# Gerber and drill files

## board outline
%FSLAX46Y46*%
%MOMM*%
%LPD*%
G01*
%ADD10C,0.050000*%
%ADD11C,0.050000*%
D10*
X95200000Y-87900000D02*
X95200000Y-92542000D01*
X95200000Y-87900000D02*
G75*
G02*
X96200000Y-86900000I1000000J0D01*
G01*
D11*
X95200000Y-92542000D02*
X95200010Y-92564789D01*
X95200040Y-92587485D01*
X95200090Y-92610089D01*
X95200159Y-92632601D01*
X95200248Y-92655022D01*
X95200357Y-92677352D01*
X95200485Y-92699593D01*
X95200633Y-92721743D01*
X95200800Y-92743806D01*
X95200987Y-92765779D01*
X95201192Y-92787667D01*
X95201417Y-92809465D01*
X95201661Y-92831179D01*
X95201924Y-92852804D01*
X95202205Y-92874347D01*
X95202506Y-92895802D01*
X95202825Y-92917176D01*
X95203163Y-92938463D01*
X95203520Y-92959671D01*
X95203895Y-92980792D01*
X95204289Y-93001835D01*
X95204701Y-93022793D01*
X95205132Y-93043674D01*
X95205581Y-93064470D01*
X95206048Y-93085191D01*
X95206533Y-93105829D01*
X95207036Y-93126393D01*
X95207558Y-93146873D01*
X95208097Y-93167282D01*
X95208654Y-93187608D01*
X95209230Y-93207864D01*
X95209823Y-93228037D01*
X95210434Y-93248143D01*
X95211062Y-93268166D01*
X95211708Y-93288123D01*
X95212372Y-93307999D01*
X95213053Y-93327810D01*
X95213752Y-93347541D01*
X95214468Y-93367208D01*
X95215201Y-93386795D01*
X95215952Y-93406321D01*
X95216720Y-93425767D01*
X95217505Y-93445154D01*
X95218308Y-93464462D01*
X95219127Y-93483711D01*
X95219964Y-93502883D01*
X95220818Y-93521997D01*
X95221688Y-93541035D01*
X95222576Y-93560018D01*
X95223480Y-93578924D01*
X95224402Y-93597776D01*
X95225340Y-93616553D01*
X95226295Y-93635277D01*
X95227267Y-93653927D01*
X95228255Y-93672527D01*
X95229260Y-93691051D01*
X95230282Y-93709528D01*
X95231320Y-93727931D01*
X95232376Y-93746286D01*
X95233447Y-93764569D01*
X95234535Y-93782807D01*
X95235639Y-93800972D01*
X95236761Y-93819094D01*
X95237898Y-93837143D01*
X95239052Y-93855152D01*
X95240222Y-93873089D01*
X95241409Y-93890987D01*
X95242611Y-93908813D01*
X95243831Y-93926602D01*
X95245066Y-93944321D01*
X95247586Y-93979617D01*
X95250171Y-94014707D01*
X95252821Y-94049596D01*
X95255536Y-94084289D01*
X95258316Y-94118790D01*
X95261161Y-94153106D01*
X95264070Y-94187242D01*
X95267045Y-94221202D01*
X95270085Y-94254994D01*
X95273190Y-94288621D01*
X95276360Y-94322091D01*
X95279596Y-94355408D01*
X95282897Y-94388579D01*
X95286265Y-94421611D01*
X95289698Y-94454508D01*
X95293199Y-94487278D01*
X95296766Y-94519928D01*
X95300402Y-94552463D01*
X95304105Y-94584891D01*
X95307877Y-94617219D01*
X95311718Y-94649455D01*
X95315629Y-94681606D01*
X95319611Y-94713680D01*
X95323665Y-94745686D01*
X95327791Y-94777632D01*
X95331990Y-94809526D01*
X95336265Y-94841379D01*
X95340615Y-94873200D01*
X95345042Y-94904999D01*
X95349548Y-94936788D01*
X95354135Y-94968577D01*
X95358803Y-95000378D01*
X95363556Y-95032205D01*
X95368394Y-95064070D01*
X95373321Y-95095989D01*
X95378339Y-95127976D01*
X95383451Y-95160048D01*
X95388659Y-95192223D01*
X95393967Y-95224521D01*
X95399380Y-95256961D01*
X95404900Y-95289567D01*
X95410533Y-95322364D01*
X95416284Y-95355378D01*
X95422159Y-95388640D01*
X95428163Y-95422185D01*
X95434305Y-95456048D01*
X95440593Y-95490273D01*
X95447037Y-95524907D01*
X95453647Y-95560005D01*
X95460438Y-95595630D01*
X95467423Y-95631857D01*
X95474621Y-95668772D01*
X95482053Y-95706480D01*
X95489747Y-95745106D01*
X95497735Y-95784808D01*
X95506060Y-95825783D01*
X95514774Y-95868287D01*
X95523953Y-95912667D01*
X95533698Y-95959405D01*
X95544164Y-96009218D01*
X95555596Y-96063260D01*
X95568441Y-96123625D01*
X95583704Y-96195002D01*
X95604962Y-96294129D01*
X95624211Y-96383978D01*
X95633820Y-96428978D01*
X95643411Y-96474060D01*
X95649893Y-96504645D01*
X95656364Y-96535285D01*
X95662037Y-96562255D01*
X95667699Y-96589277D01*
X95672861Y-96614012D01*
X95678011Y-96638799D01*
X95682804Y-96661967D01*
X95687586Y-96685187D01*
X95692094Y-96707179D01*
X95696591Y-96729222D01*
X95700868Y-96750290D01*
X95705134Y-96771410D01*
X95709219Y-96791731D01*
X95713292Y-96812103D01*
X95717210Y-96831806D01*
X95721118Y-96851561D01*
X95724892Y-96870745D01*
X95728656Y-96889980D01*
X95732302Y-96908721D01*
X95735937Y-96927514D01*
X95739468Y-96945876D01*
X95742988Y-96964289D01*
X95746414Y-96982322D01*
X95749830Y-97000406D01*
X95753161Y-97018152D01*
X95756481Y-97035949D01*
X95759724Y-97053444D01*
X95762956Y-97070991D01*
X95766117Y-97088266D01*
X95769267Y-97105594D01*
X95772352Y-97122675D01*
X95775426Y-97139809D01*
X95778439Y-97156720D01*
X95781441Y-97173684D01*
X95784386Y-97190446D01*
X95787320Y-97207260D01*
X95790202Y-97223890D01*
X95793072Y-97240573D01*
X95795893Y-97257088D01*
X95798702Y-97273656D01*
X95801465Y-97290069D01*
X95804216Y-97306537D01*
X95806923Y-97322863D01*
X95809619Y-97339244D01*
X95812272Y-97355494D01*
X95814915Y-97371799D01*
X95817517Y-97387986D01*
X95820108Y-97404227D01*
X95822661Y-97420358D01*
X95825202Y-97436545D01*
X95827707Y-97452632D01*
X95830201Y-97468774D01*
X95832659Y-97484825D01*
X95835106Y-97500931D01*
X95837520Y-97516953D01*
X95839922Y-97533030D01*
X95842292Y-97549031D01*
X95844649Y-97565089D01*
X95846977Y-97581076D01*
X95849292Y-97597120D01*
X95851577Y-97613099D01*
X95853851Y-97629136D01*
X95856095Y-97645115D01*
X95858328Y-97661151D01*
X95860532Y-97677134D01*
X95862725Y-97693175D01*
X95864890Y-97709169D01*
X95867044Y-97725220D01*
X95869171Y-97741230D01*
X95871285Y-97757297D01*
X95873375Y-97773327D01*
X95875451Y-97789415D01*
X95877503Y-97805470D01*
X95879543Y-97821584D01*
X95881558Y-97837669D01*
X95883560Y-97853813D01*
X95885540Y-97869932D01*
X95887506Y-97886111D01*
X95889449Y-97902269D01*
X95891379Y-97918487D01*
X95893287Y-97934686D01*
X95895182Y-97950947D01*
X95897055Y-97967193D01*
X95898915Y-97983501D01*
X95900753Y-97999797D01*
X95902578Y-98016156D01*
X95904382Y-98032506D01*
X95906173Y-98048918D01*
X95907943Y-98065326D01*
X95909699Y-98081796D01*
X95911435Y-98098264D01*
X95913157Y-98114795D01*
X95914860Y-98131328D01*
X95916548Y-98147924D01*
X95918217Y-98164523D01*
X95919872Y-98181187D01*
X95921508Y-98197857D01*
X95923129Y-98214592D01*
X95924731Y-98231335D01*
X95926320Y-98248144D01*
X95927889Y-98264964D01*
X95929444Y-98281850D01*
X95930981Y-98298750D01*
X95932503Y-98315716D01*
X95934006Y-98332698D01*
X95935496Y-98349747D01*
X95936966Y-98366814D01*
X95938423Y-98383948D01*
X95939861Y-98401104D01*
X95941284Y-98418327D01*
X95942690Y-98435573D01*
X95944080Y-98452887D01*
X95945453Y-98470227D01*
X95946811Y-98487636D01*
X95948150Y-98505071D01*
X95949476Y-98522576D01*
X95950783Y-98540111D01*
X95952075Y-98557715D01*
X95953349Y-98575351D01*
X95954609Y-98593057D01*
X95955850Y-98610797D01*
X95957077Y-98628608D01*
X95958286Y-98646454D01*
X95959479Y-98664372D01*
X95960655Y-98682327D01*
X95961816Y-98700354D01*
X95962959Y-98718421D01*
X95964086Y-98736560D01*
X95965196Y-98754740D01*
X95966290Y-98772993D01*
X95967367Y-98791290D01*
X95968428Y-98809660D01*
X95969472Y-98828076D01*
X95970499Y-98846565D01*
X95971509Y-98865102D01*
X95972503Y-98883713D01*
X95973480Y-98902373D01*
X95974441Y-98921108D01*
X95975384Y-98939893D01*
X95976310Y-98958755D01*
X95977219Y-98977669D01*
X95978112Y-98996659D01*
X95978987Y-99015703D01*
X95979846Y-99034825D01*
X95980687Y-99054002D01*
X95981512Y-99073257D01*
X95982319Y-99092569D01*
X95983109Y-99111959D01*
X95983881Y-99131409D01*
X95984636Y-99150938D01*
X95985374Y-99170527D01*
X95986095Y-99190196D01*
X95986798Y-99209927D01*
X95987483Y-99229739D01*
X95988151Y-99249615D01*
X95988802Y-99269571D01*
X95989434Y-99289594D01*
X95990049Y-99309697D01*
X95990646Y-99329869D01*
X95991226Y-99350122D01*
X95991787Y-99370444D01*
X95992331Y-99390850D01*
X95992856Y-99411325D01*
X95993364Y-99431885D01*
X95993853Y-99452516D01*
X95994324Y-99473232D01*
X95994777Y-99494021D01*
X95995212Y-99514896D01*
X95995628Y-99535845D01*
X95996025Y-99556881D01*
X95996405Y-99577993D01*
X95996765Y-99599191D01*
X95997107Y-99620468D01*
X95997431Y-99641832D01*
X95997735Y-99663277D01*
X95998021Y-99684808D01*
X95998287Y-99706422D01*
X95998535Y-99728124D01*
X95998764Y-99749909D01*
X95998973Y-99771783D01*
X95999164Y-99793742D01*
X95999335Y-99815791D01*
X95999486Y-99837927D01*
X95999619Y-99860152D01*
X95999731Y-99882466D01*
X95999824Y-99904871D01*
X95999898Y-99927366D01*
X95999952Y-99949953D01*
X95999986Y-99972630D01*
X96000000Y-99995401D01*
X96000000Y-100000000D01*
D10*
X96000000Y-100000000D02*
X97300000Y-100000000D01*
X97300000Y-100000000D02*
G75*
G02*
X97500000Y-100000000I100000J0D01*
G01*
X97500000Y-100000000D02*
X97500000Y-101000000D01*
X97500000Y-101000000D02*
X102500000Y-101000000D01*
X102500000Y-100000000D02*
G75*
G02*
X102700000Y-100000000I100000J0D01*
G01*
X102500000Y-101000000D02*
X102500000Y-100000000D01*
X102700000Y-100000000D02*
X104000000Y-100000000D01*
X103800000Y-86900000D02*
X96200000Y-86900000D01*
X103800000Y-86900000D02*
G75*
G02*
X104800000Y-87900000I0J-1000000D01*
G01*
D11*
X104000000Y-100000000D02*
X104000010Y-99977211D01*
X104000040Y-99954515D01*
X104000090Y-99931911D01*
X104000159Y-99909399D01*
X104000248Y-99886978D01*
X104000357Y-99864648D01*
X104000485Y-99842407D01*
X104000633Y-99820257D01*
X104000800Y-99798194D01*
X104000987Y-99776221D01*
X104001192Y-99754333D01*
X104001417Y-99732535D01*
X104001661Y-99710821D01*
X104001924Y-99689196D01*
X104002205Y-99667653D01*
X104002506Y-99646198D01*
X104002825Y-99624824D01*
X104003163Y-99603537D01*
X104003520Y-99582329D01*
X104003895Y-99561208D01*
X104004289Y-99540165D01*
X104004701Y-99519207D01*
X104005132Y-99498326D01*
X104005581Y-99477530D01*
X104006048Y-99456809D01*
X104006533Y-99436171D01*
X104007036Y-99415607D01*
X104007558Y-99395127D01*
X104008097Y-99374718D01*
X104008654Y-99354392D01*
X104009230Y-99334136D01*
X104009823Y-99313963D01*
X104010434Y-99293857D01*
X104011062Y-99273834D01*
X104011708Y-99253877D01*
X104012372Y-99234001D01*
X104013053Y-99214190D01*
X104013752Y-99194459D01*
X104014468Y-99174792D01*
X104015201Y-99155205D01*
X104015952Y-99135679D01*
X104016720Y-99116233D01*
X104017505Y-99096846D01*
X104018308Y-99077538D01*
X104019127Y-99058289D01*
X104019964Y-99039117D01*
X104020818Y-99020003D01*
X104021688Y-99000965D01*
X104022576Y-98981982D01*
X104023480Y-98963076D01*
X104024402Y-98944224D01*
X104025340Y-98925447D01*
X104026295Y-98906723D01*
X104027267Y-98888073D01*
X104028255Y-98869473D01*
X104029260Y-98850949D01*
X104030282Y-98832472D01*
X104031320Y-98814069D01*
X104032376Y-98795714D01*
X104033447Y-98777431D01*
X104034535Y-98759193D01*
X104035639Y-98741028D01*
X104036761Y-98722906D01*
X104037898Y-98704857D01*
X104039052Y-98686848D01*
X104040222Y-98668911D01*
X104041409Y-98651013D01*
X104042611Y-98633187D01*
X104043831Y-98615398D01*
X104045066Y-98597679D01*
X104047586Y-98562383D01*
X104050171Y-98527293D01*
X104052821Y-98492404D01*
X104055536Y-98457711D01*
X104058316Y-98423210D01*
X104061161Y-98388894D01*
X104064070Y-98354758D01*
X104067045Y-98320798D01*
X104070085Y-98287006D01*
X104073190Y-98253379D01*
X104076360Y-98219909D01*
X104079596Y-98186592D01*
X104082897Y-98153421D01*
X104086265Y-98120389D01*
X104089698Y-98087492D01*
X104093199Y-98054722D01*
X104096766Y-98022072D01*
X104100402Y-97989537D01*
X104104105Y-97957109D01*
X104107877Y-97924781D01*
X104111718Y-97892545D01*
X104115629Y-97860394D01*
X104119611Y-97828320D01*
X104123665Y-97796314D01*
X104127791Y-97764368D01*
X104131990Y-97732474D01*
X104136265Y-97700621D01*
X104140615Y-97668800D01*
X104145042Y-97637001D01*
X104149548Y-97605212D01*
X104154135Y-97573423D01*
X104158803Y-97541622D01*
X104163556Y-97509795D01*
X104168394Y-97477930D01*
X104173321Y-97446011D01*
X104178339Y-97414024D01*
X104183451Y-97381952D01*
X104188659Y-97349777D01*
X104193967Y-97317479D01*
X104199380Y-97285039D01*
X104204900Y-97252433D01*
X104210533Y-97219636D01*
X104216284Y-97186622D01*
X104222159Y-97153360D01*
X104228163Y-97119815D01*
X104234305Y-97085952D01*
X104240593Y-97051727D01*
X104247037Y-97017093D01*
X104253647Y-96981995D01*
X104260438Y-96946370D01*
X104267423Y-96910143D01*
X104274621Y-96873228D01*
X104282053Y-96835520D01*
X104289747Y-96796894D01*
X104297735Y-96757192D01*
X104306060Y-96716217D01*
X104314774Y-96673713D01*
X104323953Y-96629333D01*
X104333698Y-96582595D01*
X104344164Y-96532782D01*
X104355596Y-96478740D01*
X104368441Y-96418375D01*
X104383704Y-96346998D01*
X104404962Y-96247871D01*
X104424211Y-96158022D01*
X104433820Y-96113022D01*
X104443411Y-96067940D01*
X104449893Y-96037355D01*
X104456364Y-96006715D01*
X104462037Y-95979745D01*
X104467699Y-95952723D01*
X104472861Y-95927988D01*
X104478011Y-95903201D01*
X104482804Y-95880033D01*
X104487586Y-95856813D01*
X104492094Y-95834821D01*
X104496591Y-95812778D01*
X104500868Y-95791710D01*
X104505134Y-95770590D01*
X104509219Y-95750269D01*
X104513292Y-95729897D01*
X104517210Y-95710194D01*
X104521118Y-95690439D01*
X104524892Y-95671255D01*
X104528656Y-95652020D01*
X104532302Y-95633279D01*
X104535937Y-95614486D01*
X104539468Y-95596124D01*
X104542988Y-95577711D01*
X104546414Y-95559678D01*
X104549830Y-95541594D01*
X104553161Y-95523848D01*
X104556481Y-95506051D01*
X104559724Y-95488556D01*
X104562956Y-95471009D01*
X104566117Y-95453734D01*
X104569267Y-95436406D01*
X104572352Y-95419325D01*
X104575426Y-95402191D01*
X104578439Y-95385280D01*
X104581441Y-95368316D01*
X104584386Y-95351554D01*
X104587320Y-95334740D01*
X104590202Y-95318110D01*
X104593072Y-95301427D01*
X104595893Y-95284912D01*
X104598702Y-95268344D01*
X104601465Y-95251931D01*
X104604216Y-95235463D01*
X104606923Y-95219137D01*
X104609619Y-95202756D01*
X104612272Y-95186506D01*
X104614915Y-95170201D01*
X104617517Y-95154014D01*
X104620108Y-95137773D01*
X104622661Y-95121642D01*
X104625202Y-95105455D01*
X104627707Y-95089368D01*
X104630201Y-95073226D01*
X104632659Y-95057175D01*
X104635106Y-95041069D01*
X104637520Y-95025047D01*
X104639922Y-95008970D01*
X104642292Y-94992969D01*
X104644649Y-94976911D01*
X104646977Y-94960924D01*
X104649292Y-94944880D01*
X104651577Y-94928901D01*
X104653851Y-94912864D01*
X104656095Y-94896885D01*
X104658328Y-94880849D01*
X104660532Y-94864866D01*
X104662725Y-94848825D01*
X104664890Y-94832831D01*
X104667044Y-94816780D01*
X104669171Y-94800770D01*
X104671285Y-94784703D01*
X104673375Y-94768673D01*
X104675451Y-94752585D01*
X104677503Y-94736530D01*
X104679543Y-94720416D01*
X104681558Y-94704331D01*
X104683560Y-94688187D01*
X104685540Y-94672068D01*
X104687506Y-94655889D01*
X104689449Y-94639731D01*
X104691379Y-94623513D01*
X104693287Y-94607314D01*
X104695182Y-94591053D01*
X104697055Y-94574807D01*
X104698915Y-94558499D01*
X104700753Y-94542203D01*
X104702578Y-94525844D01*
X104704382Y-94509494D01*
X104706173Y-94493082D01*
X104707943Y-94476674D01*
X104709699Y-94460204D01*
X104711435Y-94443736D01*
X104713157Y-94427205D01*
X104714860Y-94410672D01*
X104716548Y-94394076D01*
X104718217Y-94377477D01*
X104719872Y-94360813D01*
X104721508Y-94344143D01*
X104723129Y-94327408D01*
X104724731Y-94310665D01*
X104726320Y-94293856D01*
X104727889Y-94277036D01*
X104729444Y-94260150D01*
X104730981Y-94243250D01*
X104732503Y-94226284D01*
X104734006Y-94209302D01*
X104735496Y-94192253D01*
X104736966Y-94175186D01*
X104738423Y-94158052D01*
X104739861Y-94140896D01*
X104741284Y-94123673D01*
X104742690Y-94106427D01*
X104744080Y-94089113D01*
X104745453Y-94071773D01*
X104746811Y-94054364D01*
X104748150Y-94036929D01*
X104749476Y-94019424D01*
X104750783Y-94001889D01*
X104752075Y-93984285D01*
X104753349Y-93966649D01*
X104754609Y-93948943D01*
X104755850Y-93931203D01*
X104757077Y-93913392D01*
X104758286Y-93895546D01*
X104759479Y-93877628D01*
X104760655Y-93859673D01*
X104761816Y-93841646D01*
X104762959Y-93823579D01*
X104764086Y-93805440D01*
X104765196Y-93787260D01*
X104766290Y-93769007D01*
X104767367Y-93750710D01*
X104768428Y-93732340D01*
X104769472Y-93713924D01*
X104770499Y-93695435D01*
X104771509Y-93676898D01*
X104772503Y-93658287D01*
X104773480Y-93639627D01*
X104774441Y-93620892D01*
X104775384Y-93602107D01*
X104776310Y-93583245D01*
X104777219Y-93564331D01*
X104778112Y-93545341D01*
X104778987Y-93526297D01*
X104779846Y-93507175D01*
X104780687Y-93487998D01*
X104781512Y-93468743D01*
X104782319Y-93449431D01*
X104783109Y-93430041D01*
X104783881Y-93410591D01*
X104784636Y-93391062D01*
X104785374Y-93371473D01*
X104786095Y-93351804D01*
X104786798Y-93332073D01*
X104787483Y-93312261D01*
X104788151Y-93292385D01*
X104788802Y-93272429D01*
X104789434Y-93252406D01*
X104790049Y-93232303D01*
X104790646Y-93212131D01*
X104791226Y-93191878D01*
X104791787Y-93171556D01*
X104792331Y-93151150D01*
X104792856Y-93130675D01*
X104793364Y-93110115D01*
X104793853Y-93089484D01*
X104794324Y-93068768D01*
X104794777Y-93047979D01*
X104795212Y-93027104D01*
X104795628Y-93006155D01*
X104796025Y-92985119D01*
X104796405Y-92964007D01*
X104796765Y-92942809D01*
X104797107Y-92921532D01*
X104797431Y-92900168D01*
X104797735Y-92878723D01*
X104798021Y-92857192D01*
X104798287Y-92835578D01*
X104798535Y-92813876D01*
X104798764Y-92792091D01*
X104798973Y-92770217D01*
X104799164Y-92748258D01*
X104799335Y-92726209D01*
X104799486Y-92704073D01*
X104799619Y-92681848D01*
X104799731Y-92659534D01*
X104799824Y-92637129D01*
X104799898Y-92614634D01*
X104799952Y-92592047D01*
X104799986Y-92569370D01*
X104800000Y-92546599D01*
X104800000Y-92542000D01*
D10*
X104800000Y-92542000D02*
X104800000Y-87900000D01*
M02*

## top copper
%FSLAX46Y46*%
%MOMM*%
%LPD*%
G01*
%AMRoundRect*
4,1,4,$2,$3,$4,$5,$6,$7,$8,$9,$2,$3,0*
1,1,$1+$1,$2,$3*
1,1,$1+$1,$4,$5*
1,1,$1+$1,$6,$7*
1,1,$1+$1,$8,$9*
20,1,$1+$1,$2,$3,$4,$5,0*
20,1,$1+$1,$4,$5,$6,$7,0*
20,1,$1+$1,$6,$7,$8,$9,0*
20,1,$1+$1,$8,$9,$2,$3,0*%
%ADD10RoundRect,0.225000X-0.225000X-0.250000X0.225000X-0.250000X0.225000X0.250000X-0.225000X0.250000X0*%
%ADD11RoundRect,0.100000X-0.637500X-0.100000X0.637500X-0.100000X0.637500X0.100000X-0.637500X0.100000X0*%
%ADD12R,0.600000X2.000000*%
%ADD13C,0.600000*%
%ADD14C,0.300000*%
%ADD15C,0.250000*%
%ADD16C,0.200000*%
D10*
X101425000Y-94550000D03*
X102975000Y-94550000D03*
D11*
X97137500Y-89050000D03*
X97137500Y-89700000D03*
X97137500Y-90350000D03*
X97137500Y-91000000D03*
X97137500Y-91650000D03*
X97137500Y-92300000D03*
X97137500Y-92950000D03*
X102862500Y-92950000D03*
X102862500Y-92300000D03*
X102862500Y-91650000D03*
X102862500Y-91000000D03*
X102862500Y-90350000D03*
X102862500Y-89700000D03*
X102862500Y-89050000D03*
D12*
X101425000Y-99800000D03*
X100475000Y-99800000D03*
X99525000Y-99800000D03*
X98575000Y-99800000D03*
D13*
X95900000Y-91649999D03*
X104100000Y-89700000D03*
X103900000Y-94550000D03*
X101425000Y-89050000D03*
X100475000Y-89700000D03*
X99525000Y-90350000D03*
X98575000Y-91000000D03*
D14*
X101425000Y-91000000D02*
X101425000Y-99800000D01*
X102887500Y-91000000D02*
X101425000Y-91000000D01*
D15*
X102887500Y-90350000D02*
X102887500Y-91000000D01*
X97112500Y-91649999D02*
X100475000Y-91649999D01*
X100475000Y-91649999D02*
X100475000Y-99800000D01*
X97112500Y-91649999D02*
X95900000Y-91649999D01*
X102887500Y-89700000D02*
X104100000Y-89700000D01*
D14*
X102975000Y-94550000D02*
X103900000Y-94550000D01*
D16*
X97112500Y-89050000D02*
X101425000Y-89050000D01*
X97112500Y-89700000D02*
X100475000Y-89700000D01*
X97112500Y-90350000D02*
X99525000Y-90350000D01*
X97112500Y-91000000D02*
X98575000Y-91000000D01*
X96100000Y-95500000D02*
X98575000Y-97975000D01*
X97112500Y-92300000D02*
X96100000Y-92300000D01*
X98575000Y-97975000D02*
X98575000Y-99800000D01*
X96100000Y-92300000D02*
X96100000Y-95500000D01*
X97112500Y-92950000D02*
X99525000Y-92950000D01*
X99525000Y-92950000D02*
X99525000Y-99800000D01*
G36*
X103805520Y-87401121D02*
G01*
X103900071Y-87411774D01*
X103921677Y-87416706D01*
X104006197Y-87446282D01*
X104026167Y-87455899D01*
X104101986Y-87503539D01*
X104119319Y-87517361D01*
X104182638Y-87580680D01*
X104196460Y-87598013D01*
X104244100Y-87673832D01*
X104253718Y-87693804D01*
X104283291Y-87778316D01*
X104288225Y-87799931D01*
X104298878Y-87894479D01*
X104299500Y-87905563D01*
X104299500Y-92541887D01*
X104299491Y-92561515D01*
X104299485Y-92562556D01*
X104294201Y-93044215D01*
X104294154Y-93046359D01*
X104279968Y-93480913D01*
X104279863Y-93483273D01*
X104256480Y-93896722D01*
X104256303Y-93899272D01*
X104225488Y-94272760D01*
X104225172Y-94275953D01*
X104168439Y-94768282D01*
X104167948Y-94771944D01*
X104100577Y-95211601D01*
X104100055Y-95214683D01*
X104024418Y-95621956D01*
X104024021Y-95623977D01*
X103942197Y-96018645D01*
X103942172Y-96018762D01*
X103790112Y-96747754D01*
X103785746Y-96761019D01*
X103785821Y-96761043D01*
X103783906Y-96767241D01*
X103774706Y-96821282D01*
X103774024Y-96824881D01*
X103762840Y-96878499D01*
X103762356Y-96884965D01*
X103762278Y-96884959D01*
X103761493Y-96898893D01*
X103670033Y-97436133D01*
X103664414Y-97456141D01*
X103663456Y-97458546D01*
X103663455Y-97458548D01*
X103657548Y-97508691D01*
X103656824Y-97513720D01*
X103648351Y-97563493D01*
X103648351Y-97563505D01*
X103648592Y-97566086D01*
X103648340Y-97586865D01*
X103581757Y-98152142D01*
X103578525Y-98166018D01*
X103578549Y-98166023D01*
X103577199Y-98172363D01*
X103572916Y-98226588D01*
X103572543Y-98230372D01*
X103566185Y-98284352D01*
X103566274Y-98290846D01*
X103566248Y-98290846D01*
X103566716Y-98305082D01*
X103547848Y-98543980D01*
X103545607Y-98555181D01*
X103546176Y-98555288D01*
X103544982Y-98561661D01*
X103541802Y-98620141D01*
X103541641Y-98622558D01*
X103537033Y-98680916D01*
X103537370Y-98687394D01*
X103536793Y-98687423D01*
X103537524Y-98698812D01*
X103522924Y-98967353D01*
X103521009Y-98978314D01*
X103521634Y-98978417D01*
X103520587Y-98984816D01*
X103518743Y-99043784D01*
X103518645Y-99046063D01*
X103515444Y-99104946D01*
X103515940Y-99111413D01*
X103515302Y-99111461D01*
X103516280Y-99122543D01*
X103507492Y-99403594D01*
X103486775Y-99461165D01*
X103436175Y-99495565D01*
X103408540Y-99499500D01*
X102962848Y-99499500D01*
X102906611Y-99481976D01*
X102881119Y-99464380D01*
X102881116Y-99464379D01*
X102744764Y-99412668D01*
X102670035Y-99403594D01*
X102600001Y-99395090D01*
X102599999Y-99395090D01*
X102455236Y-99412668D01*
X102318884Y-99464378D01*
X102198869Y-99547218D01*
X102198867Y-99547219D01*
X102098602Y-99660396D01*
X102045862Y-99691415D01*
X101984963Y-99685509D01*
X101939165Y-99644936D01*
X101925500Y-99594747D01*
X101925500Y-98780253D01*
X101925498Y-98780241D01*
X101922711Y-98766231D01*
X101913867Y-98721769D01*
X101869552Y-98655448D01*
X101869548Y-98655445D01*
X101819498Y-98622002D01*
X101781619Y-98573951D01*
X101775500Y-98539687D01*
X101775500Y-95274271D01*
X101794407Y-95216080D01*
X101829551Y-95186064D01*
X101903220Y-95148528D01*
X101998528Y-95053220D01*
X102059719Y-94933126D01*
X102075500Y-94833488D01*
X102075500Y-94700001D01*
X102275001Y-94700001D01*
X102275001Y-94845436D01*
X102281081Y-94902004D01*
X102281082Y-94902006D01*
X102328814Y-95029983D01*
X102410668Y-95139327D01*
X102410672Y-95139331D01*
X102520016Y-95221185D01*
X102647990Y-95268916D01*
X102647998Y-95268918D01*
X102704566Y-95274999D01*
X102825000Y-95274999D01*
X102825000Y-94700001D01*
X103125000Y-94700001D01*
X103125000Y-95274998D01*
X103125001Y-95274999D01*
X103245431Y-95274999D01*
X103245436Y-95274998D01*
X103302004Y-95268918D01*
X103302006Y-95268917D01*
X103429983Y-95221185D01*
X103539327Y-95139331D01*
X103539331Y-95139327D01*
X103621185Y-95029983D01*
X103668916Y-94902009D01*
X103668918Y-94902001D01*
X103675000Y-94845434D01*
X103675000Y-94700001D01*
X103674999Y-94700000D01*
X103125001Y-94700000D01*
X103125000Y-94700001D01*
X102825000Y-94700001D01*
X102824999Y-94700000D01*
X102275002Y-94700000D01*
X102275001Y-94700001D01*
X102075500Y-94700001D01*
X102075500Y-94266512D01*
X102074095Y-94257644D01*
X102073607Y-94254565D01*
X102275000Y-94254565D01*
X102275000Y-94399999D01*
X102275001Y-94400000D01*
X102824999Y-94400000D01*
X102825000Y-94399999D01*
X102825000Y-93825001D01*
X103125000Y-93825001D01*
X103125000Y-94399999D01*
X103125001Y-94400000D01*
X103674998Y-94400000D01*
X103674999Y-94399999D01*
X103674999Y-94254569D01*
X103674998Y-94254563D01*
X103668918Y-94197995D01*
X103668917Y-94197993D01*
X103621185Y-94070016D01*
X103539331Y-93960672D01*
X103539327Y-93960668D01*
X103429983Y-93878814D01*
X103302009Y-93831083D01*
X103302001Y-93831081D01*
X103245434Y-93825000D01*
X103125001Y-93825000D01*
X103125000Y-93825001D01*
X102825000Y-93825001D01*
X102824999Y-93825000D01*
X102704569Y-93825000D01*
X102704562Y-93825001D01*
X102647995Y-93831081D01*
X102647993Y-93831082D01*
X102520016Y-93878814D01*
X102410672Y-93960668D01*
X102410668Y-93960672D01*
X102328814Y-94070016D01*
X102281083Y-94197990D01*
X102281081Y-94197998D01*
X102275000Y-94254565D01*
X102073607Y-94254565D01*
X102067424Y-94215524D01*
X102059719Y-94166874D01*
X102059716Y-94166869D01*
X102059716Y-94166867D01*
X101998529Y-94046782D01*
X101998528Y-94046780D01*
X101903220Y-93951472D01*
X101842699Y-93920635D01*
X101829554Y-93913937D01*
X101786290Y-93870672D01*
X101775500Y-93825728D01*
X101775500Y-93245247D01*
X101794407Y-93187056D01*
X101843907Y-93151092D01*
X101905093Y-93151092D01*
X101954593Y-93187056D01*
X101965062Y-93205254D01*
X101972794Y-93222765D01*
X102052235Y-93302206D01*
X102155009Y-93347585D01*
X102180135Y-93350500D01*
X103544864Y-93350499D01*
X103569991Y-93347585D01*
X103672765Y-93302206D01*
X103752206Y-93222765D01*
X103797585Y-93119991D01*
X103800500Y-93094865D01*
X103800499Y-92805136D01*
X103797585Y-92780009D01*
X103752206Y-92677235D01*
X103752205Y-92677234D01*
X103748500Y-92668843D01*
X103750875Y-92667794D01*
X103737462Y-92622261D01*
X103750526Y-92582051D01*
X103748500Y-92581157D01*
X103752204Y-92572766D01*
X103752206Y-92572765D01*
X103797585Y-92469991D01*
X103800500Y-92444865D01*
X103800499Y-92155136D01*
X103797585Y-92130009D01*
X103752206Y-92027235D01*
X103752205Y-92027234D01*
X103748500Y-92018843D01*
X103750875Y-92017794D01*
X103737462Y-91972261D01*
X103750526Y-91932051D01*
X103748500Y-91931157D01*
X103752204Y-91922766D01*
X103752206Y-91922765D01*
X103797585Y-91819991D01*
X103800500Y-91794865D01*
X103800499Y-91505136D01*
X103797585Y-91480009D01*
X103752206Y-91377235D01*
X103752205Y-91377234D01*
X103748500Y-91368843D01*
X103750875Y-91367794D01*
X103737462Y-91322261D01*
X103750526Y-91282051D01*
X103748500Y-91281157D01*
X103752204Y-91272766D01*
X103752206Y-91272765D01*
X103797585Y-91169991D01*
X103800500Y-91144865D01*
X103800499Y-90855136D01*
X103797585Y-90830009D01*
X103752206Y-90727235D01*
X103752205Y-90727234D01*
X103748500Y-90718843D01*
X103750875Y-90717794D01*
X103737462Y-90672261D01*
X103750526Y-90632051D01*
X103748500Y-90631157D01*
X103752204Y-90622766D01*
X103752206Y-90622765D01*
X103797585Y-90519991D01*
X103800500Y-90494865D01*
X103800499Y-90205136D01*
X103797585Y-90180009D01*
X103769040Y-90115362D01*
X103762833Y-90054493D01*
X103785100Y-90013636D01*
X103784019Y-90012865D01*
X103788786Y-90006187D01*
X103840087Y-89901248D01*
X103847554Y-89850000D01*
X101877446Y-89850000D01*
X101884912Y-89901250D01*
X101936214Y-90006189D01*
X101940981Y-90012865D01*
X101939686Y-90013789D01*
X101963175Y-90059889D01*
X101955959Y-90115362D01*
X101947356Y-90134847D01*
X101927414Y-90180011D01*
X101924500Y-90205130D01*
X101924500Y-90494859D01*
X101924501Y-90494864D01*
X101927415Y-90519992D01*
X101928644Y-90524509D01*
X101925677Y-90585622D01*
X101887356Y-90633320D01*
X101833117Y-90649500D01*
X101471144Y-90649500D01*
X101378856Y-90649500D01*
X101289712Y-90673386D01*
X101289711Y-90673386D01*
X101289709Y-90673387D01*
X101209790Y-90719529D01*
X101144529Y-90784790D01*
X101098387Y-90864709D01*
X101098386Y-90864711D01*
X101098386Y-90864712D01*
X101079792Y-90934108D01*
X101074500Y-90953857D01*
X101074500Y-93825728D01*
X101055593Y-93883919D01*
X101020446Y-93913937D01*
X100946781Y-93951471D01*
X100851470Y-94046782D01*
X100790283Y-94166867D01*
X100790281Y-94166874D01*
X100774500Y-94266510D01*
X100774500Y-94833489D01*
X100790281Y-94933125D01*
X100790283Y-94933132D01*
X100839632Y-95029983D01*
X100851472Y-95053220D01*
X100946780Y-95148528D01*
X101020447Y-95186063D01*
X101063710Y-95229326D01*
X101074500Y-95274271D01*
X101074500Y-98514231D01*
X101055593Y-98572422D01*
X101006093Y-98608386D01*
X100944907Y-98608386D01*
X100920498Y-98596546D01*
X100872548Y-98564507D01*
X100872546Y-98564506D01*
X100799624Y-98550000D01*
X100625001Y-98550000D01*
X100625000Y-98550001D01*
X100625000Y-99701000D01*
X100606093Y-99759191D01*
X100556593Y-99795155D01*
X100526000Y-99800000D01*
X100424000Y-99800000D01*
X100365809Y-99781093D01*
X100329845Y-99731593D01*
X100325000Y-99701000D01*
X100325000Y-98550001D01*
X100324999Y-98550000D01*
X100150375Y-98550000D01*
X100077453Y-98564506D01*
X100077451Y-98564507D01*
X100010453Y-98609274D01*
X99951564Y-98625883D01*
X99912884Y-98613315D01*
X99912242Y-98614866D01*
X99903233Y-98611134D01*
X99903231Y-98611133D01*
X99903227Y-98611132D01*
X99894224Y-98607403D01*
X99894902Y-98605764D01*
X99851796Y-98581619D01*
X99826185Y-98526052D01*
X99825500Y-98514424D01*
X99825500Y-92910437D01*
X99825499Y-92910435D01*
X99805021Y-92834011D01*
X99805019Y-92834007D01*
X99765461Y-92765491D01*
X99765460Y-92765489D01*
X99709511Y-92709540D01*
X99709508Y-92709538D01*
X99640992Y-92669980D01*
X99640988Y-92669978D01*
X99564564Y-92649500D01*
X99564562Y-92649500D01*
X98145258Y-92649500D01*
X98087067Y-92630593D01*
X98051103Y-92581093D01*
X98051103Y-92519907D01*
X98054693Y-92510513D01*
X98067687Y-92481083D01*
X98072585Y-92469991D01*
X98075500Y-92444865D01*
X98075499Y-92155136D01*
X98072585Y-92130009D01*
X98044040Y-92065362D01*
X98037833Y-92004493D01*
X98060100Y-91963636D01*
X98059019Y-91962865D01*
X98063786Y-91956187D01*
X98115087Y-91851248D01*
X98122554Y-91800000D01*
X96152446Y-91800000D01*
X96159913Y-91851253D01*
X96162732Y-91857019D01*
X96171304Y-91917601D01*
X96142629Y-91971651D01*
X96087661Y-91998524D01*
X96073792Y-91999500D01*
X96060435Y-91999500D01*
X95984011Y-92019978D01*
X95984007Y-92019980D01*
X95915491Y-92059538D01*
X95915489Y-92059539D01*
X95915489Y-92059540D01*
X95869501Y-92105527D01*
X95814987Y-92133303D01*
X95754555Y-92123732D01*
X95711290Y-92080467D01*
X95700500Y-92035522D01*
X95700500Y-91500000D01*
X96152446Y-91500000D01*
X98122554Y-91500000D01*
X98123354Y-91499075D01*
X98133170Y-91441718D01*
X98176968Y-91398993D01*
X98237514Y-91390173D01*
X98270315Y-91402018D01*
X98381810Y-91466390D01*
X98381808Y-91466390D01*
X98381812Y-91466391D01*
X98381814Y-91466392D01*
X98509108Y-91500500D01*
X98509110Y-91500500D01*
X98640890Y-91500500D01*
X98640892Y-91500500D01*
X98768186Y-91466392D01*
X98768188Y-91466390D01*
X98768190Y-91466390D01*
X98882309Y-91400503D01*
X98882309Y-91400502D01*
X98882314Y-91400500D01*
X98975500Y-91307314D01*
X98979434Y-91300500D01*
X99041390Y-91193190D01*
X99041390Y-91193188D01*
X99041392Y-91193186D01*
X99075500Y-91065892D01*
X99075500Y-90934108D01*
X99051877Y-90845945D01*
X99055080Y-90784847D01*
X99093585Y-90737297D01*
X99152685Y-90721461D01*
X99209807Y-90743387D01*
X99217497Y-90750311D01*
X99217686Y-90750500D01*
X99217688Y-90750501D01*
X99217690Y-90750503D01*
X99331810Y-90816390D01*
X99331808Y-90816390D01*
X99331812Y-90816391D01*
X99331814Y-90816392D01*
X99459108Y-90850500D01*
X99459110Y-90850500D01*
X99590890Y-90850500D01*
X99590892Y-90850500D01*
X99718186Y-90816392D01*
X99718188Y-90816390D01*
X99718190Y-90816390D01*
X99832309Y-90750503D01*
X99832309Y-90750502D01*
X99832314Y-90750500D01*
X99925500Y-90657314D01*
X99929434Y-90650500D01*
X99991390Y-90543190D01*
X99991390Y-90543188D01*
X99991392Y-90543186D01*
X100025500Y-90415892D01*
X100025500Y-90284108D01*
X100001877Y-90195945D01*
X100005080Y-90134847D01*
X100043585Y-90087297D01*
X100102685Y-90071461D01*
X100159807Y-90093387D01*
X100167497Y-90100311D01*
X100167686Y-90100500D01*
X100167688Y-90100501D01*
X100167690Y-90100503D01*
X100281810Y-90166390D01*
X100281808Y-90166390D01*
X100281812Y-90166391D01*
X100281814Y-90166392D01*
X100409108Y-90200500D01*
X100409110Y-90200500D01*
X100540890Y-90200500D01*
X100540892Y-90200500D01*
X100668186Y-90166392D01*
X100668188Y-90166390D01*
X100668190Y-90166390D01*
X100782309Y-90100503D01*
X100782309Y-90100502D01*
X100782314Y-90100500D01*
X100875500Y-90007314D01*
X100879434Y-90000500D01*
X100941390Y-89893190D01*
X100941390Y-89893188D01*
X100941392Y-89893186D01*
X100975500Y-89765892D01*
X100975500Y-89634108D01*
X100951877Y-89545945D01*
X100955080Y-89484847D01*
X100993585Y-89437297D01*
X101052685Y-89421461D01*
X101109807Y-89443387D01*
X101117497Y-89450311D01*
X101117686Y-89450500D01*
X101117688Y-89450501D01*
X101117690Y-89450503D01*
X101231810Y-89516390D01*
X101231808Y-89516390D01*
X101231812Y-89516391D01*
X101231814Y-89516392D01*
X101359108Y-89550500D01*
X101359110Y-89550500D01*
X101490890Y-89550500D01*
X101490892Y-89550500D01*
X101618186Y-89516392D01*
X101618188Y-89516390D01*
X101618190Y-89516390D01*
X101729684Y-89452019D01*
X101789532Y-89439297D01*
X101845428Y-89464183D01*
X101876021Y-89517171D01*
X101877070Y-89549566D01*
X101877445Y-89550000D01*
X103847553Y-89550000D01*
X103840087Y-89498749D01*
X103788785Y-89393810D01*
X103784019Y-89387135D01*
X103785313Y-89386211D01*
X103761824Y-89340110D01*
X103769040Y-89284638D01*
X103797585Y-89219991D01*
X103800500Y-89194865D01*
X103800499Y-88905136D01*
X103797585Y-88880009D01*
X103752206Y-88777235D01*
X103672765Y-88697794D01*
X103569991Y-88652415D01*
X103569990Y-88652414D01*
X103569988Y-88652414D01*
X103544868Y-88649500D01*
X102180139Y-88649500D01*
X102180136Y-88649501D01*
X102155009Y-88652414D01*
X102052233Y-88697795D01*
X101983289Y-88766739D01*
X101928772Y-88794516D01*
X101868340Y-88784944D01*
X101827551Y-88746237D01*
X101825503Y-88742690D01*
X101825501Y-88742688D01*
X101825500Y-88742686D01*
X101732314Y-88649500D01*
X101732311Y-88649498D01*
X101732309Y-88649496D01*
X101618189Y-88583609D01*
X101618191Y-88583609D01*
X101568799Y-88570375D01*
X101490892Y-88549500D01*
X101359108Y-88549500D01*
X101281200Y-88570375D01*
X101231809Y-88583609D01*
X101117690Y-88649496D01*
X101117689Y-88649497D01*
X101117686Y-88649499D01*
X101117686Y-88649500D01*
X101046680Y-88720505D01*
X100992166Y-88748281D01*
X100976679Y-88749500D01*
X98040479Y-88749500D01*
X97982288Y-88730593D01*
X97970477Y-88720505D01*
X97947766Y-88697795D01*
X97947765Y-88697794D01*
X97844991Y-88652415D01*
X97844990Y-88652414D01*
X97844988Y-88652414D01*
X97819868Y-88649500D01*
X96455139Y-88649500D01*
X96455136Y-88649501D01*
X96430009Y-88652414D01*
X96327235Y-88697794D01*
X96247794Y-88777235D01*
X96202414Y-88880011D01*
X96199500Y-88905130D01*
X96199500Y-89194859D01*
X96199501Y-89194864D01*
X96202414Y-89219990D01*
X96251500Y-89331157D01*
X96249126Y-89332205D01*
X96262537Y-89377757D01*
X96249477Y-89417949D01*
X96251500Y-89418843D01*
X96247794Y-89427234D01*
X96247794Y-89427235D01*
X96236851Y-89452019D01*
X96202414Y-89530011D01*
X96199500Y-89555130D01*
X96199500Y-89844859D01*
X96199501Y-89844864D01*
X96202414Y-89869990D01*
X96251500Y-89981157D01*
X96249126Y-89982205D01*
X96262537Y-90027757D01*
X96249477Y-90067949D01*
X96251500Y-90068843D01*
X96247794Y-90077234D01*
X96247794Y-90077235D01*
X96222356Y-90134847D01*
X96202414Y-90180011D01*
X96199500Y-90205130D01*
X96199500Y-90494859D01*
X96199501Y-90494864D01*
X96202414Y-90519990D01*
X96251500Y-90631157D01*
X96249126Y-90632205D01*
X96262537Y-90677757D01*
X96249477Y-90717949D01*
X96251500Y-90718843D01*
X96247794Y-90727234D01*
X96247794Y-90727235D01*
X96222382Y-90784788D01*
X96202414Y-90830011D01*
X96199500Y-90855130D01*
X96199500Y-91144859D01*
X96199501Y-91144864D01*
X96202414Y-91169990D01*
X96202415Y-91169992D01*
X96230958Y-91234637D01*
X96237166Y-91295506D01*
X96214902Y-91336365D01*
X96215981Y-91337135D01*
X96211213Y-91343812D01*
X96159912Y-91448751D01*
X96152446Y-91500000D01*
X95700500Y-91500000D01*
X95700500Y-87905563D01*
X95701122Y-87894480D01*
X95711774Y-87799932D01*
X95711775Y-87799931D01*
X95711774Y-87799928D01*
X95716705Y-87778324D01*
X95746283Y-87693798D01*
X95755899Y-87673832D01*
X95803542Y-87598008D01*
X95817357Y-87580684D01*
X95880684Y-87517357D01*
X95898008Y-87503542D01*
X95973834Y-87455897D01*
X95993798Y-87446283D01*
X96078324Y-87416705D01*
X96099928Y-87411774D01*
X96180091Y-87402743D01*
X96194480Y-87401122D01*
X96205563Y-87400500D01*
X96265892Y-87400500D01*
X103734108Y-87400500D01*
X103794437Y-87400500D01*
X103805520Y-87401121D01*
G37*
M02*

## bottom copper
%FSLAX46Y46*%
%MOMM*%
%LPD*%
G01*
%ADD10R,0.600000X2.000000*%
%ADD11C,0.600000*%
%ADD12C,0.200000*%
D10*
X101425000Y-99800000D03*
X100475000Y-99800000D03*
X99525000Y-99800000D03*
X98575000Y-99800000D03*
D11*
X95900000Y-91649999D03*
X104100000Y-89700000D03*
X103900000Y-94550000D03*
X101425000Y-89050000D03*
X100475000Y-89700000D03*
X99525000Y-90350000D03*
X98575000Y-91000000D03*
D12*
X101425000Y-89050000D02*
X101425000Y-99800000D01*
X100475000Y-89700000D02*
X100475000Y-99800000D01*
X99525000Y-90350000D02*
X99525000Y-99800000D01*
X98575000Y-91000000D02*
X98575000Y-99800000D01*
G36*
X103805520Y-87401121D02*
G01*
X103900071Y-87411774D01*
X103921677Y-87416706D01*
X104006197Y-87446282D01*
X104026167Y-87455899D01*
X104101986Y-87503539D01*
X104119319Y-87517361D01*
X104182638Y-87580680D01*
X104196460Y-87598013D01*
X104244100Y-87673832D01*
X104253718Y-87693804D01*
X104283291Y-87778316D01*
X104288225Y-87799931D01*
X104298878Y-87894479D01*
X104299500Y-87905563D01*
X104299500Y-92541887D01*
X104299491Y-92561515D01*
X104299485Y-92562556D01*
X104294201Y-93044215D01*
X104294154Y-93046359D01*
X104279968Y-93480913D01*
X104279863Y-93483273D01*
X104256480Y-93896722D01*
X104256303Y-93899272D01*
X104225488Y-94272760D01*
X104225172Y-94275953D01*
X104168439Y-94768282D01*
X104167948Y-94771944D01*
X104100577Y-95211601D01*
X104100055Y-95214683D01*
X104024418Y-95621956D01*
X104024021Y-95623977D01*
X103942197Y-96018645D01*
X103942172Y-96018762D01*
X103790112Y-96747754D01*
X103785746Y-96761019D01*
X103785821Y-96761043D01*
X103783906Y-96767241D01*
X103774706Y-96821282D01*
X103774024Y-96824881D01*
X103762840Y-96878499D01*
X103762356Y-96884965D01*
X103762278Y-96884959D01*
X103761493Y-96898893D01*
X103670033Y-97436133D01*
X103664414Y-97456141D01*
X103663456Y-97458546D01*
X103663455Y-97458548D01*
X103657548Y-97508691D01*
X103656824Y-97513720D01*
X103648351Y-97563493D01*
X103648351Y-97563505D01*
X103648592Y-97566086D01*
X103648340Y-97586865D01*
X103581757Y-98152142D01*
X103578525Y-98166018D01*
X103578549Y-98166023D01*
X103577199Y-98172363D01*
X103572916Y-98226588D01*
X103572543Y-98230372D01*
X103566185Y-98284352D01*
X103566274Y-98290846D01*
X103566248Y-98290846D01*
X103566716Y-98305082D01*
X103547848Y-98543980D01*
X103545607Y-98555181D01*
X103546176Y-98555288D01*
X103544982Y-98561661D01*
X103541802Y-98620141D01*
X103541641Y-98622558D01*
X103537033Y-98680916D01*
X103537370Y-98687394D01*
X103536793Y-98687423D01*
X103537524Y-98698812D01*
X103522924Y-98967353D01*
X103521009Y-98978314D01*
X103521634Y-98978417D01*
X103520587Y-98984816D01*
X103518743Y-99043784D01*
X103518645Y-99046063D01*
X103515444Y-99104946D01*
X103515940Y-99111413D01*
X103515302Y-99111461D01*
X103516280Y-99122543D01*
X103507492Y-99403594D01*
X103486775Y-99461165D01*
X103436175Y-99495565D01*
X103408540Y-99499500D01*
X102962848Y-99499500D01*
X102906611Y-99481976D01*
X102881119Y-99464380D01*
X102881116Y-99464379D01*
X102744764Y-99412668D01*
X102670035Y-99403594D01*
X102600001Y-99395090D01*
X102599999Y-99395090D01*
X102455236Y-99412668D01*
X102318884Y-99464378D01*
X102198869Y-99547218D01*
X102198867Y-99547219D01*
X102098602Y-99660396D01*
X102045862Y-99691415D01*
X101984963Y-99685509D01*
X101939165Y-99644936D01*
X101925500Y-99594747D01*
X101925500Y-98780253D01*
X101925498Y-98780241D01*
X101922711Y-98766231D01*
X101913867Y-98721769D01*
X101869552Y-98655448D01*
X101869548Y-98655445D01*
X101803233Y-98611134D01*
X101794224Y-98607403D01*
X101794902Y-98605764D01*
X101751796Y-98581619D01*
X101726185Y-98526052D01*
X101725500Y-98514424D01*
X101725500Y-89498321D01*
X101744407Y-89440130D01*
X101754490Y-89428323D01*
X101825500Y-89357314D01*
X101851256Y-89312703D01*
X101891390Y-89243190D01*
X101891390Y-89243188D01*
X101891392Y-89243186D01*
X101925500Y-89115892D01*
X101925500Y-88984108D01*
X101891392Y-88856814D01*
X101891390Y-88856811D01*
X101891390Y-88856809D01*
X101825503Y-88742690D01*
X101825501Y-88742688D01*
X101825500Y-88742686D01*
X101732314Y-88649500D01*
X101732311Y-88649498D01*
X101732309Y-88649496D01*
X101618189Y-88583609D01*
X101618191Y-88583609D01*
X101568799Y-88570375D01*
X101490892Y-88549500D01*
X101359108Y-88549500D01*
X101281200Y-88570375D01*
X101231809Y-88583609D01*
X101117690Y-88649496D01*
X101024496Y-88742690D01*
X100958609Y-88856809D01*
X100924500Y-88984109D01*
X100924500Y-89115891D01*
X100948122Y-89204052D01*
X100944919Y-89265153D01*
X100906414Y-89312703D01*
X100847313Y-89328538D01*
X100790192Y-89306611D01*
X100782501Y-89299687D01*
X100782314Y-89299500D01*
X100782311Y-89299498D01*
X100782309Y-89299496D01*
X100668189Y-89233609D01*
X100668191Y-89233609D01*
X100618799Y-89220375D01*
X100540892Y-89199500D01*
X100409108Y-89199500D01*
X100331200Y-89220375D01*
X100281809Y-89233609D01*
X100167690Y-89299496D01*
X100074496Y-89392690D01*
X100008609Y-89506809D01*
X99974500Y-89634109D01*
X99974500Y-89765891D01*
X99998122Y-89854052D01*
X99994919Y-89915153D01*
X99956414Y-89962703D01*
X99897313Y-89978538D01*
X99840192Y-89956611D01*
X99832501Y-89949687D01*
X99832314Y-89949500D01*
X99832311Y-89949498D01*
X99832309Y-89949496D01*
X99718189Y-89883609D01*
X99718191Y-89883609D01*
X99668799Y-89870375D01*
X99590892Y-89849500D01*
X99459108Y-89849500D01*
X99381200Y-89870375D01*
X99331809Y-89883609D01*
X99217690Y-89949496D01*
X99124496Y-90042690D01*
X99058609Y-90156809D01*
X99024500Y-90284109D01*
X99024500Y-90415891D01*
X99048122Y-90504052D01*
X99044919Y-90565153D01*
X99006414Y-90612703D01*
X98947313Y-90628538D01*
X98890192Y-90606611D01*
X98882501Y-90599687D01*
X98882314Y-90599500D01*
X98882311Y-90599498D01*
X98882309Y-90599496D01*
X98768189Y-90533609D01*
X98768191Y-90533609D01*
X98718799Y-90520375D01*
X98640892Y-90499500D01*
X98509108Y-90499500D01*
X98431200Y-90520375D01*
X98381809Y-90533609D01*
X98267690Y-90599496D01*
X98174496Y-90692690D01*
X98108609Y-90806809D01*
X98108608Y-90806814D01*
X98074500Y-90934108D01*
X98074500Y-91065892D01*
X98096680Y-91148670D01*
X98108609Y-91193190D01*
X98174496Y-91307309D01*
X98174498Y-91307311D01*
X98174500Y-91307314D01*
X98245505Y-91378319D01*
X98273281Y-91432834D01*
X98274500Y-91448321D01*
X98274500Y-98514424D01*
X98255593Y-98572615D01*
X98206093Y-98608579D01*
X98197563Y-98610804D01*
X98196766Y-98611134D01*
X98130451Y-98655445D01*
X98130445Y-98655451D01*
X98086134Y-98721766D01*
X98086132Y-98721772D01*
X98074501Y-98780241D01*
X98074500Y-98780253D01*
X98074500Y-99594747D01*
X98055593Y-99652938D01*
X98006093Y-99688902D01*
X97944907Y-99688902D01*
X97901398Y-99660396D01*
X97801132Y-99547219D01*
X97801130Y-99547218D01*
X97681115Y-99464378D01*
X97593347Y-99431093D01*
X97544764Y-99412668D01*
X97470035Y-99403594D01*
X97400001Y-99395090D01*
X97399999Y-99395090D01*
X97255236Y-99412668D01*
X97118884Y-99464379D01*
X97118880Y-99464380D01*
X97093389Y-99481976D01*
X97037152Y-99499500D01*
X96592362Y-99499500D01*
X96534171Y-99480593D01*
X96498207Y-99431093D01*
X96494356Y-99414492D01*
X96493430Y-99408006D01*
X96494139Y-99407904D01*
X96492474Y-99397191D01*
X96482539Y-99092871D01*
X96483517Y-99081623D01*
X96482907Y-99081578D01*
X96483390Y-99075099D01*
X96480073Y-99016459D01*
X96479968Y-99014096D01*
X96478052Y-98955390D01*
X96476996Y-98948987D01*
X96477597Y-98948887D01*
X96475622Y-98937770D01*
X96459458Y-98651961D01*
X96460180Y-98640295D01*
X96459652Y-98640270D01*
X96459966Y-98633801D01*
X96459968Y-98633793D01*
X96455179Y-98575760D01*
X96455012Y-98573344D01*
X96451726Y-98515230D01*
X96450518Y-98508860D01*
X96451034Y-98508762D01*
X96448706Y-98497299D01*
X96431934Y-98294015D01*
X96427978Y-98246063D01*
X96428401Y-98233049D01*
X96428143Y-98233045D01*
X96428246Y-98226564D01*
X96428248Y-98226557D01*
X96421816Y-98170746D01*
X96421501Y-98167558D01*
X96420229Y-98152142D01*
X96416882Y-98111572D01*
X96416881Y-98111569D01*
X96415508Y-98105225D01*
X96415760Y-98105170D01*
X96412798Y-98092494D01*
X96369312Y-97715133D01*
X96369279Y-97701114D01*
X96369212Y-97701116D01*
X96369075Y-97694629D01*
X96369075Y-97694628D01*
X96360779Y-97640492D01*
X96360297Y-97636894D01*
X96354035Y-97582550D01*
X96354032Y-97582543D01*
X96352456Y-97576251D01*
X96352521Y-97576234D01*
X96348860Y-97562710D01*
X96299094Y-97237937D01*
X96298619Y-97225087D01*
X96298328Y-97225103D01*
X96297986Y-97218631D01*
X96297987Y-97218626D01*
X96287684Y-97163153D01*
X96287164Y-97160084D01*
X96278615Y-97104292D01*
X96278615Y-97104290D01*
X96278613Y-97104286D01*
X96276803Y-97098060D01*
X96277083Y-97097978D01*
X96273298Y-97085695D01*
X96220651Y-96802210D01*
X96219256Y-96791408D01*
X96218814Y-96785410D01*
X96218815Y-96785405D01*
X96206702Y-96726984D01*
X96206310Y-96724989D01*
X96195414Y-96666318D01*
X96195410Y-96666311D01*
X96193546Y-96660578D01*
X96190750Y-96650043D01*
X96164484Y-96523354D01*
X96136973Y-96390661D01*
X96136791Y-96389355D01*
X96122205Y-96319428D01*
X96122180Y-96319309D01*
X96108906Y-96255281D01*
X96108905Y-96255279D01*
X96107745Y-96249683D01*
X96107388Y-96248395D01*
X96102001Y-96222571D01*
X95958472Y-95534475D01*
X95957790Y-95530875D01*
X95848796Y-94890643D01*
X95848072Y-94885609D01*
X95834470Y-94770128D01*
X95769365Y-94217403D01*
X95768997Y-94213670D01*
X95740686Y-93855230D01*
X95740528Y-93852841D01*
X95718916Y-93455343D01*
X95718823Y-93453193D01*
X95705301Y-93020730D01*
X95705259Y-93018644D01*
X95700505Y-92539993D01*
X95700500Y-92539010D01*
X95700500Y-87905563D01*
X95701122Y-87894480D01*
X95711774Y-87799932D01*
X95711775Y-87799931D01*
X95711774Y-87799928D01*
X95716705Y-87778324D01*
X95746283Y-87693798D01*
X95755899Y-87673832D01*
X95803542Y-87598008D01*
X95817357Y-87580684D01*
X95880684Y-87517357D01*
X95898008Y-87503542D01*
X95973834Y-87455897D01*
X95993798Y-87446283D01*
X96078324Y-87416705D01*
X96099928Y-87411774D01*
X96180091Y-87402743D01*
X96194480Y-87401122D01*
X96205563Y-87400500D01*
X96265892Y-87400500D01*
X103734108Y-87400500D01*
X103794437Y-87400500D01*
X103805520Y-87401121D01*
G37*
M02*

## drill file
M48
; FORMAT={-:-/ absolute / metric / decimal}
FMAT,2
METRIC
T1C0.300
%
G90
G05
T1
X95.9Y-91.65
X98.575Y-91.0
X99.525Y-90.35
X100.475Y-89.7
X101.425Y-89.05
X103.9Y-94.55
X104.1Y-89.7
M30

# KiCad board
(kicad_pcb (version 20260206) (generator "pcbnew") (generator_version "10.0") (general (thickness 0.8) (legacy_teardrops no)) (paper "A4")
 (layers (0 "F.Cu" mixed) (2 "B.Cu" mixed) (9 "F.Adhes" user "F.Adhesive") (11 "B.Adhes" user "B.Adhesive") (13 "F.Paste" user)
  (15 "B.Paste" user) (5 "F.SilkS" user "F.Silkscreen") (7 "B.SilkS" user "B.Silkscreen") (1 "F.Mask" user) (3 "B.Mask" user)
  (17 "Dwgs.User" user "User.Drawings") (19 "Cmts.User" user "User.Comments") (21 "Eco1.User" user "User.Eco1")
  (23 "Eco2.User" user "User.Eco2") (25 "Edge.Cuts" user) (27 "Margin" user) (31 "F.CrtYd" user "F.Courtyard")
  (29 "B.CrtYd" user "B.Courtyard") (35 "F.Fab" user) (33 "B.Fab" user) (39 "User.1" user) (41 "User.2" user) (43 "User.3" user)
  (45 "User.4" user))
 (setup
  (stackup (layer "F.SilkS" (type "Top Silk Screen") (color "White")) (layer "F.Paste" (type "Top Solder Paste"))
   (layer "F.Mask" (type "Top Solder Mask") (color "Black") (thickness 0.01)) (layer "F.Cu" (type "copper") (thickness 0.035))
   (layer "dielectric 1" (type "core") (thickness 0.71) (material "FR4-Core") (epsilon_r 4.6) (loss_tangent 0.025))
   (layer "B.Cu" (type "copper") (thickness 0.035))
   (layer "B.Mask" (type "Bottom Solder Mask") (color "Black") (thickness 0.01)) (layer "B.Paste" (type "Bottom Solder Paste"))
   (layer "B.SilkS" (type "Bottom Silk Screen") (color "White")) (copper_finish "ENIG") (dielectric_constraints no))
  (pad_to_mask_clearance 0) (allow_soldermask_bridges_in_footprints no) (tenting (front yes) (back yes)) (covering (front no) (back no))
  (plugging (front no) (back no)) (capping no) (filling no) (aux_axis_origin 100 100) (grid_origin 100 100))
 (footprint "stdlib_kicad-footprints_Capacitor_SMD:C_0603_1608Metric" (layer "F.Cu") (at 102.2 94.55)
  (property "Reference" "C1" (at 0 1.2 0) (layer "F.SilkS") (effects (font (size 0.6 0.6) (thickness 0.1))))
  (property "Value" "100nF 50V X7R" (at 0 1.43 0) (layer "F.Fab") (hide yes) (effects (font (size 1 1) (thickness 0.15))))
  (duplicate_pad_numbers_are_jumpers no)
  (pad "1" smd roundrect (at -0.775 0) (size 0.9 0.95) (layers "F.Cu" "F.Mask" "F.Paste") (roundrect_rratio 0.25) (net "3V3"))
  (pad "2" smd roundrect (at 0.775 0) (size 0.9 0.95) (layers "F.Cu" "F.Mask" "F.Paste") (roundrect_rratio 0.25) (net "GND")))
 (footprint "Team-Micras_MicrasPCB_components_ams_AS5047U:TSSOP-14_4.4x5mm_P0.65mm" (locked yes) (layer "F.Cu") (at 100 91)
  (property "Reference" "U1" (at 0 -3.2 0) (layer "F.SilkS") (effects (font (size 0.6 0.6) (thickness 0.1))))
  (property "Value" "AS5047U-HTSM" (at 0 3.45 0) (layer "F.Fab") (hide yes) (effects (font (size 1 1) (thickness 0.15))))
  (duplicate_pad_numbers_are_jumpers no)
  (pad "1" smd roundrect (at -2.8625 -1.95) (size 1.475 0.4) (layers "F.Cu" "F.Mask" "F.Paste") (roundrect_rratio 0.25) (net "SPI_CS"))
  (pad "2" smd roundrect (at -2.8625 -1.3) (size 1.475 0.4) (layers "F.Cu" "F.Mask" "F.Paste") (roundrect_rratio 0.25) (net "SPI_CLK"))
  (pad "3" smd roundrect (at -2.8625 -0.65) (size 1.475 0.4) (layers "F.Cu" "F.Mask" "F.Paste") (roundrect_rratio 0.25) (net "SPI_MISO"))
  (pad "4" smd roundrect (at -2.8625 0) (size 1.475 0.4) (layers "F.Cu" "F.Mask" "F.Paste") (roundrect_rratio 0.25) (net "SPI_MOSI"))
  (pad "5" smd roundrect (at -2.8625 0.65) (size 1.475 0.4) (layers "F.Cu" "F.Mask" "F.Paste") (roundrect_rratio 0.25) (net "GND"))
  (pad "6" smd roundrect (at -2.8625 1.3) (size 1.475 0.4) (layers "F.Cu" "F.Mask" "F.Paste") (roundrect_rratio 0.25) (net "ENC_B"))
  (pad "7" smd roundrect (at -2.8625 1.95) (size 1.475 0.4) (layers "F.Cu" "F.Mask" "F.Paste") (roundrect_rratio 0.25) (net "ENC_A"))
  (pad "8" smd roundrect (at 2.8625 1.95) (size 1.475 0.4) (layers "F.Cu" "F.Mask" "F.Paste") (roundrect_rratio 0.25)
   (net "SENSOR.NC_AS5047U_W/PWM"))
  (pad "9" smd roundrect (at 2.8625 1.3) (size 1.475 0.4) (layers "F.Cu" "F.Mask" "F.Paste") (roundrect_rratio 0.25)
   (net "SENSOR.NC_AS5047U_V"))
  (pad "10" smd roundrect (at 2.8625 0.65) (size 1.475 0.4) (layers "F.Cu" "F.Mask" "F.Paste") (roundrect_rratio 0.25)
   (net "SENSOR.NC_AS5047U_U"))
  (pad "11" smd roundrect (at 2.8625 0) (size 1.475 0.4) (layers "F.Cu" "F.Mask" "F.Paste") (roundrect_rratio 0.25) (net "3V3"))
  (pad "12" smd roundrect (at 2.8625 -0.65) (size 1.475 0.4) (layers "F.Cu" "F.Mask" "F.Paste") (roundrect_rratio 0.25) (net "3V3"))
  (pad "13" smd roundrect (at 2.8625 -1.3) (size 1.475 0.4) (layers "F.Cu" "F.Mask" "F.Paste") (roundrect_rratio 0.25) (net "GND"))
  (pad "14" smd roundrect (at 2.8625 -1.95) (size 1.475 0.4) (layers "F.Cu" "F.Mask" "F.Paste") (roundrect_rratio 0.25)
   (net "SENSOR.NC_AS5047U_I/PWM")))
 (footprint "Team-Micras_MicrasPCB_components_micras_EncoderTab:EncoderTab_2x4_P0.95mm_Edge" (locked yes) (layer "F.Cu") (at 100 100)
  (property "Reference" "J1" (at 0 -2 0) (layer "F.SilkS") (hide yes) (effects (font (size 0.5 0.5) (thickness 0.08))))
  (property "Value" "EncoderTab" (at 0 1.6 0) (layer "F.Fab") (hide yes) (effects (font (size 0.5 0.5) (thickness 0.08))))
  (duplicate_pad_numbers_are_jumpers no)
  (pad "1" smd rect (at 1.425 -0.2) (size 0.6 2) (layers "B.Cu" "B.Mask" "B.Paste") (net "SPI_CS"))
  (pad "2" smd rect (at 0.475 -0.2) (size 0.6 2) (layers "B.Cu" "B.Mask" "B.Paste") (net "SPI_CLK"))
  (pad "3" smd rect (at -0.475 -0.2) (size 0.6 2) (layers "B.Cu" "B.Mask" "B.Paste") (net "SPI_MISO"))
  (pad "4" smd rect (at -1.425 -0.2) (size 0.6 2) (layers "B.Cu" "B.Mask" "B.Paste") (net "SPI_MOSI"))
  (pad "5" smd rect (at 1.425 -0.2) (size 0.6 2) (layers "F.Cu" "F.Mask" "F.Paste") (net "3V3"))
  (pad "6" smd rect (at 0.475 -0.2) (size 0.6 2) (layers "F.Cu" "F.Mask" "F.Paste") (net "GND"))
  (pad "7" smd rect (at -0.475 -0.2) (size 0.6 2) (layers "F.Cu" "F.Mask" "F.Paste") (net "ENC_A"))
  (pad "8" smd rect (at -1.425 -0.2) (size 0.6 2) (layers "F.Cu" "F.Mask" "F.Paste") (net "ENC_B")))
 (gr_line (start 95.2 87.9) (end 95.2 92.542) (stroke (width 0.05) (type default)) (layer "Edge.Cuts"))
 (gr_arc (start 95.2 87.9) (mid 95.492893 87.192893) (end 96.2 86.9) (stroke (width 0.05) (type default)) (layer "Edge.Cuts"))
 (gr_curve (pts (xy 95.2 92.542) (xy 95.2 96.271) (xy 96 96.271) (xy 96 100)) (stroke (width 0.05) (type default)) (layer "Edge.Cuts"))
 (gr_line (start 96 100) (end 97.3 100) (stroke (width 0.05) (type default)) (layer "Edge.Cuts"))
 (gr_arc (start 97.3 100) (mid 97.4 99.9) (end 97.5 100) (stroke (width 0.05) (type default)) (layer "Edge.Cuts"))
 (gr_line (start 97.5 100) (end 97.5 101) (stroke (width 0.05) (type default)) (layer "Edge.Cuts"))
 (gr_line (start 97.5 101) (end 102.5 101) (stroke (width 0.05) (type default)) (layer "Edge.Cuts"))
 (gr_arc (start 102.5 100) (mid 102.6 99.9) (end 102.7 100) (stroke (width 0.05) (type default)) (layer "Edge.Cuts"))
 (gr_line (start 102.5 101) (end 102.5 100) (stroke (width 0.05) (type default)) (layer "Edge.Cuts"))
 (gr_line (start 102.7 100) (end 104 100) (stroke (width 0.05) (type default)) (layer "Edge.Cuts"))
 (gr_line (start 103.8 86.9) (end 96.2 86.9) (stroke (width 0.05) (type default)) (layer "Edge.Cuts"))
 (gr_arc (start 103.8 86.9) (mid 104.507107 87.192893) (end 104.8 87.9) (stroke (width 0.05) (type default)) (layer "Edge.Cuts"))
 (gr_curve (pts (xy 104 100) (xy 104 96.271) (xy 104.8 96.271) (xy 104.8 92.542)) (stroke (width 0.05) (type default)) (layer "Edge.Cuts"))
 (gr_line (start 104.8 92.542) (end 104.8 87.9) (stroke (width 0.05) (type default)) (layer "Edge.Cuts"))
 (segment (start 101.425 91) (end 101.425 99.8) (width 0.3) (layer "F.Cu") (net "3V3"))
 (segment (start 102.8875 91) (end 101.425 91) (width 0.3) (layer "F.Cu") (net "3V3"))
 (segment (start 102.8875 90.35) (end 102.8875 91) (width 0.25) (layer "F.Cu") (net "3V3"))
 (segment (start 97.1125 91.649999) (end 100.475 91.649999) (width 0.25) (layer "F.Cu") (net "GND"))
 (segment (start 100.475 91.649999) (end 100.475 99.8) (width 0.25) (layer "F.Cu") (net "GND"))
 (segment (start 97.1125 91.649999) (end 95.9 91.649999) (width 0.25) (layer "F.Cu") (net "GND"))
 (segment (start 102.8875 89.7) (end 104.1 89.7) (width 0.25) (layer "F.Cu") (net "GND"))
 (segment (start 102.975 94.55) (end 103.9 94.55) (width 0.3) (layer "F.Cu") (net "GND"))
 (via (at 95.9 91.649999) (size 0.6) (drill 0.3) (layers "F.Cu" "B.Cu") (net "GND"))
 (via (at 104.1 89.7) (size 0.6) (drill 0.3) (layers "F.Cu" "B.Cu") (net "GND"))
 (via (at 103.9 94.55) (size 0.6) (drill 0.3) (layers "F.Cu" "B.Cu") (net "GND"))
 (segment (start 97.1125 89.05) (end 101.425 89.05) (width 0.2) (layer "F.Cu") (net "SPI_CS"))
 (via (at 101.425 89.05) (size 0.6) (drill 0.3) (layers "F.Cu" "B.Cu") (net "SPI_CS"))
 (segment (start 101.425 89.05) (end 101.425 99.8) (width 0.2) (layer "B.Cu") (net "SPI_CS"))
 (segment (start 97.1125 89.7) (end 100.475 89.7) (width 0.2) (layer "F.Cu") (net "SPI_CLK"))
 (via (at 100.475 89.7) (size 0.6) (drill 0.3) (layers "F.Cu" "B.Cu") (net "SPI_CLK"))
 (segment (start 100.475 89.7) (end 100.475 99.8) (width 0.2) (layer "B.Cu") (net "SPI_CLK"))
 (segment (start 97.1125 90.35) (end 99.525 90.35) (width 0.2) (layer "F.Cu") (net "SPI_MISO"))
 (via (at 99.525 90.35) (size 0.6) (drill 0.3) (layers "F.Cu" "B.Cu") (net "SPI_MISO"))
 (segment (start 99.525 90.35) (end 99.525 99.8) (width 0.2) (layer "B.Cu") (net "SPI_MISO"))
 (segment (start 97.1125 91) (end 98.575 91) (width 0.2) (layer "F.Cu") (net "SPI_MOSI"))
 (via (at 98.575 91) (size 0.6) (drill 0.3) (layers "F.Cu" "B.Cu") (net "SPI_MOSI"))
 (segment (start 98.575 91) (end 98.575 99.8) (width 0.2) (layer "B.Cu") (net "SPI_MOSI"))
 (segment (start 96.1 95.5) (end 98.575 97.975) (width 0.2) (layer "F.Cu") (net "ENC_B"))
 (segment (start 97.1125 92.3) (end 96.1 92.3) (width 0.2) (layer "F.Cu") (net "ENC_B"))
 (segment (start 98.575 97.975) (end 98.575 99.8) (width 0.2) (layer "F.Cu") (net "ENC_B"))
 (segment (start 96.1 92.3) (end 96.1 95.5) (width 0.2) (layer "F.Cu") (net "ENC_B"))
 (segment (start 97.1125 92.95) (end 99.525 92.95) (width 0.2) (layer "F.Cu") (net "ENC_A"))
 (segment (start 99.525 92.95) (end 99.525 99.8) (width 0.2) (layer "F.Cu") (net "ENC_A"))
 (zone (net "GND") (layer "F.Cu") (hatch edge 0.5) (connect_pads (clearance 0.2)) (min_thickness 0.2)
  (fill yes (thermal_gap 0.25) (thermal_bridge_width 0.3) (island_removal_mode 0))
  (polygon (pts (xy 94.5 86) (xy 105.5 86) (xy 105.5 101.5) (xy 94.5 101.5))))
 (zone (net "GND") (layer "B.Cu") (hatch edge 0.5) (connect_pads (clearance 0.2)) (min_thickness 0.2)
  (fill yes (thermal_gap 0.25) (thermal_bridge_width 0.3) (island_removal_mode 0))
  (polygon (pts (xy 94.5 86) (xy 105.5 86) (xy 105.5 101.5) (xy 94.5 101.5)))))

